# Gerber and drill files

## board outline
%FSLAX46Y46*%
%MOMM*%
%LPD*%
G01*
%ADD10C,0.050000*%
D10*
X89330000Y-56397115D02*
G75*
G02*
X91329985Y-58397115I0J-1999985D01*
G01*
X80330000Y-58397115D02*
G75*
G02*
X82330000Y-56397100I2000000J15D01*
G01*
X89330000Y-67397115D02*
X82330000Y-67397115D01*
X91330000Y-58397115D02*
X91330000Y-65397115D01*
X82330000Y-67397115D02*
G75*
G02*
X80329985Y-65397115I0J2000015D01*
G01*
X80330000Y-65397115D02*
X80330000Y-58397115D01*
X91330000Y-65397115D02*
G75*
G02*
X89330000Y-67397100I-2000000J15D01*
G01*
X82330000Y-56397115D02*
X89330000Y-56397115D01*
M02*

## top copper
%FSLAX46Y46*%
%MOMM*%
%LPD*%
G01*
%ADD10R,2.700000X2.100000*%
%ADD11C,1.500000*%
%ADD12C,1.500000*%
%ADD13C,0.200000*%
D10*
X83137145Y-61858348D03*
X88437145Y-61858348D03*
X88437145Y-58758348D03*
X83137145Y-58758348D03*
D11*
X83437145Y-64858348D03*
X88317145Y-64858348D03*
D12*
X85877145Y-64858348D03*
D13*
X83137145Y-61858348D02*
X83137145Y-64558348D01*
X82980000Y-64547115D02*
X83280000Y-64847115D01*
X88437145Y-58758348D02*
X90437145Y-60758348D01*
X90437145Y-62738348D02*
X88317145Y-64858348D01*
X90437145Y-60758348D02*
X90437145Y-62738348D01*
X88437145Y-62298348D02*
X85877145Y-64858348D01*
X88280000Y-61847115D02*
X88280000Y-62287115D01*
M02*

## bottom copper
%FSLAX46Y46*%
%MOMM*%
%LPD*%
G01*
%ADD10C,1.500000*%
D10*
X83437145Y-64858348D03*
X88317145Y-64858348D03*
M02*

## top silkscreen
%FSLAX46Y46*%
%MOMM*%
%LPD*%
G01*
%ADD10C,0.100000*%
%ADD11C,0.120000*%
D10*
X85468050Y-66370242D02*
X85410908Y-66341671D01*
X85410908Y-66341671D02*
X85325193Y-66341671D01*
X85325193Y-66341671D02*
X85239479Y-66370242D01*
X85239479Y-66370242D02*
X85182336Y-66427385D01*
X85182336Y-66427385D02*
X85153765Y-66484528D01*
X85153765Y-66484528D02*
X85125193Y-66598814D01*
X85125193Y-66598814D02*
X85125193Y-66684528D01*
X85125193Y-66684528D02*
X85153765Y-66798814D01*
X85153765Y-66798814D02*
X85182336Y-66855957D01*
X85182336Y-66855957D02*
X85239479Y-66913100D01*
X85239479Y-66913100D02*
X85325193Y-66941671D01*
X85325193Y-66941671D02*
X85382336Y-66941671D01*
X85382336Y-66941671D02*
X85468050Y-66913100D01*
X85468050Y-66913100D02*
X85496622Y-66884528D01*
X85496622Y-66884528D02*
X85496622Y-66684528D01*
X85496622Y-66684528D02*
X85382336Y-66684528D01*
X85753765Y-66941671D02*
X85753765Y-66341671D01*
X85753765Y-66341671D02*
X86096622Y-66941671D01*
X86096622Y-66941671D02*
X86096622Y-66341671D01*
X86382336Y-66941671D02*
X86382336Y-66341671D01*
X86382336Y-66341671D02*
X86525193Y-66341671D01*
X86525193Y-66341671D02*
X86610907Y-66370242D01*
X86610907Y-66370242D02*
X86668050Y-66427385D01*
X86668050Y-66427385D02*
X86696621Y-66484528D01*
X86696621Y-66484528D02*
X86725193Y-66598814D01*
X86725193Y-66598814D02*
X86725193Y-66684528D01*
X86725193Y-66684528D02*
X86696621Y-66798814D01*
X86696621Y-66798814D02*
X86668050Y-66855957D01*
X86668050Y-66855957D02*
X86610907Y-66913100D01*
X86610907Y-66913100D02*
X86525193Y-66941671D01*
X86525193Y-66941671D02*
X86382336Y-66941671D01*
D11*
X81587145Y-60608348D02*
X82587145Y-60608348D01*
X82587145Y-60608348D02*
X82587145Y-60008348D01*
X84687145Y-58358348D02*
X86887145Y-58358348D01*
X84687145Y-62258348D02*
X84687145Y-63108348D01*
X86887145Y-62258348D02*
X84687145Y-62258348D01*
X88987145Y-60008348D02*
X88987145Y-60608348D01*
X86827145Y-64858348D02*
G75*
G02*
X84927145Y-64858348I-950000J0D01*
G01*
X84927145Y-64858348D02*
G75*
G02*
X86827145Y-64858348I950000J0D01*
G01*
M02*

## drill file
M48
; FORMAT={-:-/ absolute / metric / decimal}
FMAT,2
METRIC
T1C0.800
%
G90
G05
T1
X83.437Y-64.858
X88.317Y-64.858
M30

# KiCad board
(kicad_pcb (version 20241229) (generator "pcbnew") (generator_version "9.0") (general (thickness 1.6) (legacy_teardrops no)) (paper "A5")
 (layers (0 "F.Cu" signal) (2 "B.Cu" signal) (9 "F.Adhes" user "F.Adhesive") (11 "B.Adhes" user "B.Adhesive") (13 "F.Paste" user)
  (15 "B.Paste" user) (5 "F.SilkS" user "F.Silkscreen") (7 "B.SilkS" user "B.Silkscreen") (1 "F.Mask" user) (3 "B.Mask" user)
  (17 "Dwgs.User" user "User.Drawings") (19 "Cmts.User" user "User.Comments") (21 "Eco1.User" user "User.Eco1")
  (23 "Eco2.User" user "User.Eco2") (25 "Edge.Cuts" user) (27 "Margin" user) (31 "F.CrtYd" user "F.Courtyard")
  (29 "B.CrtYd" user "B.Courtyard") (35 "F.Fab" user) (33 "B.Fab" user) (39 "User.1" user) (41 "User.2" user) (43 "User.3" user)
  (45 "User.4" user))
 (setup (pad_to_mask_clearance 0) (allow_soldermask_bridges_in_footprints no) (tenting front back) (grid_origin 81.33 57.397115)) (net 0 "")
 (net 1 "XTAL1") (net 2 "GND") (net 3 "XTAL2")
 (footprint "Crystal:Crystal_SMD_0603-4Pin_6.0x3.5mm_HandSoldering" (layer "F.Cu") (at 85.787145 60.308348)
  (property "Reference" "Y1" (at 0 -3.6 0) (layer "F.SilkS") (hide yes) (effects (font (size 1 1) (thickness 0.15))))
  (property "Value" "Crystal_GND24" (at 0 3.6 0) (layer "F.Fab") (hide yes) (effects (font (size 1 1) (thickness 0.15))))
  (fp_line (start -4.2 0.3) (end -3.2 0.3) (stroke (width 0.12) (type solid)) (layer "F.SilkS"))
  (fp_line (start -3.2 0.3) (end -3.2 -0.3) (stroke (width 0.12) (type solid)) (layer "F.SilkS"))
  (fp_line (start -1.1 -1.95) (end 1.1 -1.95) (stroke (width 0.12) (type solid)) (layer "F.SilkS"))
  (fp_line (start -1.1 1.95) (end -1.1 2.8) (stroke (width 0.12) (type solid)) (layer "F.SilkS"))
  (fp_line (start 1.1 1.95) (end -1.1 1.95) (stroke (width 0.12) (type solid)) (layer "F.SilkS"))
  (fp_line (start 3.2 -0.3) (end 3.2 0.3) (stroke (width 0.12) (type solid)) (layer "F.SilkS"))
  (pad "1" smd rect (at -2.65 1.55) (size 2.7 2.1) (layers "F.Cu" "F.Mask" "F.Paste") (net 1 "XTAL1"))
  (pad "2" smd rect (at 2.65 1.55) (size 2.7 2.1) (layers "F.Cu" "F.Mask" "F.Paste") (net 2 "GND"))
  (pad "3" smd rect (at 2.65 -1.55) (size 2.7 2.1) (layers "F.Cu" "F.Mask" "F.Paste") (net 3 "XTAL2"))
  (pad "4" smd rect (at -2.65 -1.55) (size 2.7 2.1) (layers "F.Cu" "F.Mask" "F.Paste") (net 2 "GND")))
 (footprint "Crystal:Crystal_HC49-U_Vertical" (layer "F.Cu") (at 83.437145 64.858348)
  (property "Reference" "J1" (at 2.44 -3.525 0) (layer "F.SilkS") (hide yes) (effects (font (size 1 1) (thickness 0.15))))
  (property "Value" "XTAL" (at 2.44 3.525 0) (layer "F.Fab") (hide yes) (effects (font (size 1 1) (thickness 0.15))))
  (pad "1" thru_hole circle (at 0 0) (size 1.5 1.5) (drill 0.8) (layers "*.Cu" "*.Mask") (remove_unused_layers no) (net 1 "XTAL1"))
  (pad "2" thru_hole circle (at 4.88 0) (size 1.5 1.5) (drill 0.8) (layers "*.Cu" "*.Mask") (remove_unused_layers no) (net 3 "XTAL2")))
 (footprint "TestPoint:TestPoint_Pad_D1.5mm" (layer "F.Cu") (at 85.877145 64.858348)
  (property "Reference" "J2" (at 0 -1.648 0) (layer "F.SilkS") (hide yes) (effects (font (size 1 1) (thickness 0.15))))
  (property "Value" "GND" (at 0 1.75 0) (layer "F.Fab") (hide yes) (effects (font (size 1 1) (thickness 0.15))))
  (fp_circle (center 0 0) (end 0 0.95) (stroke (width 0.12) (type solid)) (fill no) (layer "F.SilkS"))
  (pad "1" smd circle (at 0 0) (size 1.5 1.5) (layers "F.Cu" "F.Mask") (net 2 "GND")))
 (gr_arc (start 89.33 56.397115) (mid 90.744214 56.982901) (end 91.33 58.397115) (stroke (width 0.05) (type default)) (layer "Edge.Cuts"))
 (gr_arc (start 80.33 58.397115) (mid 80.915781 56.982892) (end 82.33 56.397115) (stroke (width 0.05) (type default)) (layer "Edge.Cuts"))
 (gr_line (start 89.33 67.397115) (end 82.33 67.397115) (stroke (width 0.05) (type default)) (layer "Edge.Cuts"))
 (gr_line (start 91.33 58.397115) (end 91.33 65.397115) (stroke (width 0.05) (type default)) (layer "Edge.Cuts"))
 (gr_arc (start 82.33 67.397115) (mid 80.915786 66.811329) (end 80.33 65.397115) (stroke (width 0.05) (type default)) (layer "Edge.Cuts"))
 (gr_line (start 80.33 65.397115) (end 80.33 58.397115) (stroke (width 0.05) (type default)) (layer "Edge.Cuts"))
 (gr_arc (start 91.33 65.397115) (mid 90.744208 66.811319) (end 89.33 67.397115) (stroke (width 0.05) (type default)) (layer "Edge.Cuts"))
 (gr_line (start 82.33 56.397115) (end 89.33 56.397115) (stroke (width 0.05) (type default)) (layer "Edge.Cuts"))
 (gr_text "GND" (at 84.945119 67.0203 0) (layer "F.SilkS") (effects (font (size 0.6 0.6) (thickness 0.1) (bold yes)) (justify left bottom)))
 (segment (start 83.137145 61.858348) (end 83.137145 64.558348) (width 0.2) (layer "F.Cu") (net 1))
 (segment (start 82.98 64.547115) (end 83.28 64.847115) (width 0.2) (layer "F.Cu") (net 1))
 (segment (start 88.437145 58.758348) (end 90.437145 60.758348) (width 0.2) (layer "F.Cu") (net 3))
 (segment (start 90.437145 62.738348) (end 88.317145 64.858348) (width 0.2) (layer "F.Cu") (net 3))
 (segment (start 90.437145 60.758348) (end 90.437145 62.738348) (width 0.2) (layer "F.Cu") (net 3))
 (segment (start 88.437145 62.298348) (end 85.877145 64.858348) (width 0.2) (layer "F.Cu") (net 2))
 (segment (start 88.28 61.847115) (end 88.28 62.287115) (width 0.2) (layer "F.Cu") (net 2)))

